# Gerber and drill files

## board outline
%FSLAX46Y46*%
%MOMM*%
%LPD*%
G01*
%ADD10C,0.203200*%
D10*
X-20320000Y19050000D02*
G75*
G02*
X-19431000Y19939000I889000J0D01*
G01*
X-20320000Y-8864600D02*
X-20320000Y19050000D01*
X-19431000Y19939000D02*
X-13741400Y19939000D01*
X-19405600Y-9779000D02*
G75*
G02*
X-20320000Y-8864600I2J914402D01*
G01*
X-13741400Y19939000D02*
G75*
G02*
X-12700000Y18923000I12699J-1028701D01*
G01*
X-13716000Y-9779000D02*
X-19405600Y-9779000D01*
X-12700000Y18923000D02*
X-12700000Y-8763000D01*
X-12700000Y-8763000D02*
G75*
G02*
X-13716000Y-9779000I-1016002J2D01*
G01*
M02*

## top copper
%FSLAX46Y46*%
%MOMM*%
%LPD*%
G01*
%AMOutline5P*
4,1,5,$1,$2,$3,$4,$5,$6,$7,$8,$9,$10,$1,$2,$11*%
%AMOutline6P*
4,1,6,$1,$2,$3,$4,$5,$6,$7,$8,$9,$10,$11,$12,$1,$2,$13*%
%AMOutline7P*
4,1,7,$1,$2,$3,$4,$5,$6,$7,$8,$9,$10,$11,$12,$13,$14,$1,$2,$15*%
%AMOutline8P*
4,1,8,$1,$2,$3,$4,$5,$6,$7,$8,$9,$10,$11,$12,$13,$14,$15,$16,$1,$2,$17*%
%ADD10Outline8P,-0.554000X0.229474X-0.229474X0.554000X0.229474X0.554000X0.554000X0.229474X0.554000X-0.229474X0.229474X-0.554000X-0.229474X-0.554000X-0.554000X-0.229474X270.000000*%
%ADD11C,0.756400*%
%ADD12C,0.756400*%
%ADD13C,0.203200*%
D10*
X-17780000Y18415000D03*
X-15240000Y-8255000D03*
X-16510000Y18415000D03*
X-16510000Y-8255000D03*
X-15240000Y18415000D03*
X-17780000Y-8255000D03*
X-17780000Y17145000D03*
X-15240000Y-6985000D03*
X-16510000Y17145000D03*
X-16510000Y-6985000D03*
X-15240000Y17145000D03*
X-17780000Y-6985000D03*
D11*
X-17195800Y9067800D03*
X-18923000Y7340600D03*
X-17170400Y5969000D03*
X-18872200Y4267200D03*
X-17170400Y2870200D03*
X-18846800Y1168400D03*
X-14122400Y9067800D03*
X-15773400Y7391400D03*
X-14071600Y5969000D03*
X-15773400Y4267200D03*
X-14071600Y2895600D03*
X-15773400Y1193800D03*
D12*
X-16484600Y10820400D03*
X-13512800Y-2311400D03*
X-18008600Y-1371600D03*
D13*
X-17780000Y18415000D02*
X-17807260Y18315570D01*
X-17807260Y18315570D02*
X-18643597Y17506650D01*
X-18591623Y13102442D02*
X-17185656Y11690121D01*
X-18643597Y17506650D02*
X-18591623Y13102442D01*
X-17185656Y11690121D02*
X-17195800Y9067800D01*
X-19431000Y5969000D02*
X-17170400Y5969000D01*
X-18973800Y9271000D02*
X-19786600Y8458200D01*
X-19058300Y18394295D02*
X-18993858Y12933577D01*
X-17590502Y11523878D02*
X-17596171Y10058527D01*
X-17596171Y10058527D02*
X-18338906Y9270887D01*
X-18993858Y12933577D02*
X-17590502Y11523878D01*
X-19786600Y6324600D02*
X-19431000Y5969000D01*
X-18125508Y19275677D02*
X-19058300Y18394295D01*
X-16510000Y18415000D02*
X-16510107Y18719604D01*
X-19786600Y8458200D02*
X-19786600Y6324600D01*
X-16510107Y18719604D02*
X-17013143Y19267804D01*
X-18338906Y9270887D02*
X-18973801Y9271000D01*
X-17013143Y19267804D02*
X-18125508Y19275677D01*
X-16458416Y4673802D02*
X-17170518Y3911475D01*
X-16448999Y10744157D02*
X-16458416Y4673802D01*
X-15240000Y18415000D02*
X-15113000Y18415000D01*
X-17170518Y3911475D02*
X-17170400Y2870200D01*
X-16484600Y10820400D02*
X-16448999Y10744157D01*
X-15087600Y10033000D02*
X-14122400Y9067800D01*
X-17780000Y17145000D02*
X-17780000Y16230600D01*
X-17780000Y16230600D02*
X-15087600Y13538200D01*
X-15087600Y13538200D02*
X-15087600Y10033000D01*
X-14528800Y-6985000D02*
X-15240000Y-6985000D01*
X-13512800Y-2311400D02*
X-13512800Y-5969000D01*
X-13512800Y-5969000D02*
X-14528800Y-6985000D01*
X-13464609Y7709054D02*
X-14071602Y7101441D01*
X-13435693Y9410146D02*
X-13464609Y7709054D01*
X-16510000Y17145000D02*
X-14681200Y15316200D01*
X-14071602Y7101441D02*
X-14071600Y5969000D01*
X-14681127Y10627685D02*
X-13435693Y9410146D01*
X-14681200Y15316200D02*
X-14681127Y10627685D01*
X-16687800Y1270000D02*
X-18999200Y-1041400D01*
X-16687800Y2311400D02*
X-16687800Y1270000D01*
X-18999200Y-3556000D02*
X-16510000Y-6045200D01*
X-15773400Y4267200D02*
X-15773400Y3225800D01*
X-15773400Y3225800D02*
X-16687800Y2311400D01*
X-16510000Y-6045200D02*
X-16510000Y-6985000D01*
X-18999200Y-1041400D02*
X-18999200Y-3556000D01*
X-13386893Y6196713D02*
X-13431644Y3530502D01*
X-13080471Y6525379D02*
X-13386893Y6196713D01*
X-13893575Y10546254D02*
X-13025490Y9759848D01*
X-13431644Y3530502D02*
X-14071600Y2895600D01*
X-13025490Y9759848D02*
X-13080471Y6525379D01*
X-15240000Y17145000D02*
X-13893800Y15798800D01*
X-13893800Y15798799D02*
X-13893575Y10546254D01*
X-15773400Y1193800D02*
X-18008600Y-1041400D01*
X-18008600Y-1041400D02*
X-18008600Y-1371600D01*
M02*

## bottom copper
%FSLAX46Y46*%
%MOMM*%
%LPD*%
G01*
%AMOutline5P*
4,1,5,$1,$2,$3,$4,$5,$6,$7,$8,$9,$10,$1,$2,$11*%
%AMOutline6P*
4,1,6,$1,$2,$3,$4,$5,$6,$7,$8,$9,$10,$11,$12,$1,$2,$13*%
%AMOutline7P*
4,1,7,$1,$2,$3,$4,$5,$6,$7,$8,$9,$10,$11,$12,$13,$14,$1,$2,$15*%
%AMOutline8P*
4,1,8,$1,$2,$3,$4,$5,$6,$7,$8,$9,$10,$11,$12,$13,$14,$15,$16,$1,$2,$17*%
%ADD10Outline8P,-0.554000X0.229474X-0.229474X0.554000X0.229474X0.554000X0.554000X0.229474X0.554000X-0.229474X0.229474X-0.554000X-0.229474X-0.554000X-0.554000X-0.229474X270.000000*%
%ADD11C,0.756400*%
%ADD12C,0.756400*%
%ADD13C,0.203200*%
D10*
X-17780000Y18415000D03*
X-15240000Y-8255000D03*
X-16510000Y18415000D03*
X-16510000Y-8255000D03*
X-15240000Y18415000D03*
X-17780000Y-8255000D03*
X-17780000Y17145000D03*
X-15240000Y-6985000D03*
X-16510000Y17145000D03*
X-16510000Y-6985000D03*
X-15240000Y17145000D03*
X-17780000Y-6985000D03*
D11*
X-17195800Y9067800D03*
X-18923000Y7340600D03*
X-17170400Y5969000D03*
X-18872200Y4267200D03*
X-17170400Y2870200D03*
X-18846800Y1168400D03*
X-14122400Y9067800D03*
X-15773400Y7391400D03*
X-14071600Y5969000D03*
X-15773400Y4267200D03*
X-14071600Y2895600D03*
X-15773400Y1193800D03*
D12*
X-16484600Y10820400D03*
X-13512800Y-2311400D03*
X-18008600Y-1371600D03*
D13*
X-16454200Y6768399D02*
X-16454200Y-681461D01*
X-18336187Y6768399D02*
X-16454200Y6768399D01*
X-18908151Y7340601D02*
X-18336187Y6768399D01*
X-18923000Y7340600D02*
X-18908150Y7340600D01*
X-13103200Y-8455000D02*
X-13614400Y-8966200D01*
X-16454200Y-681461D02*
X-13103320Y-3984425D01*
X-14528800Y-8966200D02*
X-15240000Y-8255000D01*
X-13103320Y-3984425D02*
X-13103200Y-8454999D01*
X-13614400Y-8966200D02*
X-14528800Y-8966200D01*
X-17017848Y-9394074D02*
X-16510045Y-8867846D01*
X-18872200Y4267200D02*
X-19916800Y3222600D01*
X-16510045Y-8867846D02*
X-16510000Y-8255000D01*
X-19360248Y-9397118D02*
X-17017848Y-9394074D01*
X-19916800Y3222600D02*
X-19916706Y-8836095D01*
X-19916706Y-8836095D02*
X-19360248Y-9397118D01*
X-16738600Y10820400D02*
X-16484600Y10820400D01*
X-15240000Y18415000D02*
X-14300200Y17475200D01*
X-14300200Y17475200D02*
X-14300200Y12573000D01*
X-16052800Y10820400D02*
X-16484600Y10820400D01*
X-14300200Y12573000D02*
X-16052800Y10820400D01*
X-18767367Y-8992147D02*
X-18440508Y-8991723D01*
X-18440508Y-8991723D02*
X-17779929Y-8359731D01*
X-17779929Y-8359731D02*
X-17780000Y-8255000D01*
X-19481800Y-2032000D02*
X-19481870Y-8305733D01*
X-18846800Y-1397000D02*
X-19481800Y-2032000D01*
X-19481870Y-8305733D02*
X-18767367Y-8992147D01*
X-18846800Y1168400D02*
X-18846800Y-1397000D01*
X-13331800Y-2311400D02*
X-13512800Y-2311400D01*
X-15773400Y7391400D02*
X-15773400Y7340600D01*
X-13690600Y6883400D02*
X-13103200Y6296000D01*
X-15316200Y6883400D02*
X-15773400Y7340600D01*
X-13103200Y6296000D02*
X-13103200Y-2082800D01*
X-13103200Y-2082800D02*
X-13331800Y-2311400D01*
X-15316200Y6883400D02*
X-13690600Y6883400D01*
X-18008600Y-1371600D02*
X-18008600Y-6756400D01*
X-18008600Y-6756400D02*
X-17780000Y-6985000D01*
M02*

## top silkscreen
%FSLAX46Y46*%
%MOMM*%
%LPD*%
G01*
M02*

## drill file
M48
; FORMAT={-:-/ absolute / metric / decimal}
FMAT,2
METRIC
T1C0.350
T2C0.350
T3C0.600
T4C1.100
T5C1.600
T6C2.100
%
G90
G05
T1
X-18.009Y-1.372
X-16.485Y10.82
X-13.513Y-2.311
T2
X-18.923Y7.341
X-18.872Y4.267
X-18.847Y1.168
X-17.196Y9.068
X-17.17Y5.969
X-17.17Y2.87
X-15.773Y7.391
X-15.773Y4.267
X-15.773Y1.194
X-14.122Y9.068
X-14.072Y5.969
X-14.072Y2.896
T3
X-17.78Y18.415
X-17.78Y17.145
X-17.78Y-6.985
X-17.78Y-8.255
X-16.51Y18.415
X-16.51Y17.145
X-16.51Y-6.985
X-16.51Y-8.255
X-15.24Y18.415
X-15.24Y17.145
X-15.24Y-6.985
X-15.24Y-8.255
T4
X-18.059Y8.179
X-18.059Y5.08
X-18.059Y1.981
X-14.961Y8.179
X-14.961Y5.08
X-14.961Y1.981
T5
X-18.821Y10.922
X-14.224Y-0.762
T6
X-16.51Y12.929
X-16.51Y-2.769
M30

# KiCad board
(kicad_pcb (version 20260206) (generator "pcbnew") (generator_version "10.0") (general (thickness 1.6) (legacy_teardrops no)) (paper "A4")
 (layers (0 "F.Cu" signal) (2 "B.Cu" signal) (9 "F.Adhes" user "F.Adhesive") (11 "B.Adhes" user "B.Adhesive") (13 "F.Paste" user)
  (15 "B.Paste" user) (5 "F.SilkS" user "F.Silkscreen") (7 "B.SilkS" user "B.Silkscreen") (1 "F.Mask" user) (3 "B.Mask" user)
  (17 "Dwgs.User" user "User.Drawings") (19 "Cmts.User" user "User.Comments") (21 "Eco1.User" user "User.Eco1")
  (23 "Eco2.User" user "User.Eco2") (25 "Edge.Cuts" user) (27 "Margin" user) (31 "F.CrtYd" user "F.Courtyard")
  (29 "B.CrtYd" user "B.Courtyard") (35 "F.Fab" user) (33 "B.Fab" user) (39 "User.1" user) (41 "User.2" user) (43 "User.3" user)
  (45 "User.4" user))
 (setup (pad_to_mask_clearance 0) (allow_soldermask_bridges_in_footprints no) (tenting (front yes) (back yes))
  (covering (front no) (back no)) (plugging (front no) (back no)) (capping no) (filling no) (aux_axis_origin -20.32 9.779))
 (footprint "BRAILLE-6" (layer "F.Cu") (at -16.51 -5.08)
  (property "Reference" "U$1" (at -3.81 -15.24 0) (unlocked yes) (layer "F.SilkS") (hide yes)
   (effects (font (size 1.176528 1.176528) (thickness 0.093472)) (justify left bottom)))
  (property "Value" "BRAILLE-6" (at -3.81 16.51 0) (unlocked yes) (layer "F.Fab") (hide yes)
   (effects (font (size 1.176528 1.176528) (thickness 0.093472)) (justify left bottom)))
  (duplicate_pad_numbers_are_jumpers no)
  (pad "P$1" thru_hole roundrect (at -1.27 -13.335 270) (size 1.108 1.108) (drill 0.6) (layers "*.Cu" "*.Mask") (remove_unused_layers no)
   (roundrect_rratio 0.25) (chamfer_ratio 0.2928932188) (chamfer top_left top_right bottom_left bottom_right) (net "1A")
   (solder_mask_margin 0.025) (thermal_bridge_angle 0))
  (pad "P$2" thru_hole roundrect (at 1.27 13.335 270) (size 1.108 1.108) (drill 0.6) (layers "*.Cu" "*.Mask") (remove_unused_layers no)
   (roundrect_rratio 0.25) (chamfer_ratio 0.2928932188) (chamfer top_left top_right bottom_left bottom_right) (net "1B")
   (solder_mask_margin 0.025) (thermal_bridge_angle 0))
  (pad "P$3" thru_hole roundrect (at 0 -13.335 270) (size 1.108 1.108) (drill 0.6) (layers "*.Cu" "*.Mask") (remove_unused_layers no)
   (roundrect_rratio 0.25) (chamfer_ratio 0.2928932188) (chamfer top_left top_right bottom_left bottom_right) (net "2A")
   (solder_mask_margin 0.025) (thermal_bridge_angle 0))
  (pad "P$4" thru_hole roundrect (at 0 13.335 270) (size 1.108 1.108) (drill 0.6) (layers "*.Cu" "*.Mask") (remove_unused_layers no)
   (roundrect_rratio 0.25) (chamfer_ratio 0.2928932188) (chamfer top_left top_right bottom_left bottom_right) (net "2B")
   (solder_mask_margin 0.025) (thermal_bridge_angle 0))
  (pad "P$5" thru_hole roundrect (at 1.27 -13.335 270) (size 1.108 1.108) (drill 0.6) (layers "*.Cu" "*.Mask") (remove_unused_layers no)
   (roundrect_rratio 0.25) (chamfer_ratio 0.2928932188) (chamfer top_left top_right bottom_left bottom_right) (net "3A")
   (solder_mask_margin 0.025) (thermal_bridge_angle 0))
  (pad "P$6" thru_hole roundrect (at -1.27 13.335 270) (size 1.108 1.108) (drill 0.6) (layers "*.Cu" "*.Mask") (remove_unused_layers no)
   (roundrect_rratio 0.25) (chamfer_ratio 0.2928932188) (chamfer top_left top_right bottom_left bottom_right) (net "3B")
   (solder_mask_margin 0.025) (thermal_bridge_angle 0))
  (pad "P$7" thru_hole roundrect (at -1.27 -12.065 270) (size 1.108 1.108) (drill 0.6) (layers "*.Cu" "*.Mask") (remove_unused_layers no)
   (roundrect_rratio 0.25) (chamfer_ratio 0.2928932188) (chamfer top_left top_right bottom_left bottom_right) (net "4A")
   (solder_mask_margin 0.025) (thermal_bridge_angle 0))
  (pad "P$8" thru_hole roundrect (at 1.27 12.065 270) (size 1.108 1.108) (drill 0.6) (layers "*.Cu" "*.Mask") (remove_unused_layers no)
   (roundrect_rratio 0.25) (chamfer_ratio 0.2928932188) (chamfer top_left top_right bottom_left bottom_right) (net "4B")
   (solder_mask_margin 0.025) (thermal_bridge_angle 0))
  (pad "P$9" thru_hole roundrect (at 0 -12.065 270) (size 1.108 1.108) (drill 0.6) (layers "*.Cu" "*.Mask") (remove_unused_layers no)
   (roundrect_rratio 0.25) (chamfer_ratio 0.2928932188) (chamfer top_left top_right bottom_left bottom_right) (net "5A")
   (solder_mask_margin 0.025) (thermal_bridge_angle 0))
  (pad "P$10" thru_hole roundrect (at 0 12.065 270) (size 1.108 1.108) (drill 0.6) (layers "*.Cu" "*.Mask") (remove_unused_layers no)
   (roundrect_rratio 0.25) (chamfer_ratio 0.2928932188) (chamfer top_left top_right bottom_left bottom_right) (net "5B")
   (solder_mask_margin 0.025) (thermal_bridge_angle 0))
  (pad "P$11" thru_hole roundrect (at 1.27 -12.065 270) (size 1.108 1.108) (drill 0.6) (layers "*.Cu" "*.Mask") (remove_unused_layers no)
   (roundrect_rratio 0.25) (chamfer_ratio 0.2928932188) (chamfer top_left top_right bottom_left bottom_right) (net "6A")
   (solder_mask_margin 0.025) (thermal_bridge_angle 0))
  (pad "P$12" thru_hole roundrect (at -1.27 12.065 270) (size 1.108 1.108) (drill 0.6) (layers "*.Cu" "*.Mask") (remove_unused_layers no)
   (roundrect_rratio 0.25) (chamfer_ratio 0.2928932188) (chamfer top_left top_right bottom_left bottom_right) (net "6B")
   (solder_mask_margin 0.025) (thermal_bridge_angle 0)))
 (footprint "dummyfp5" (layer "F.Cu") (at -14.9606 -1.9812)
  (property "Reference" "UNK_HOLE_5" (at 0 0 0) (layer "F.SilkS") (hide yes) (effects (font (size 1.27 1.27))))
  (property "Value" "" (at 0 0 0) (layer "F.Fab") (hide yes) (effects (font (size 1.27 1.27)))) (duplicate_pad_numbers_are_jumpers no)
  (pad "" np_thru_hole circle (at 0 0) (size 1.1 1.1) (drill 1.1) (layers "*.Cu" "*.Mask")))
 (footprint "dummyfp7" (layer "F.Cu") (at -16.51 2.7686)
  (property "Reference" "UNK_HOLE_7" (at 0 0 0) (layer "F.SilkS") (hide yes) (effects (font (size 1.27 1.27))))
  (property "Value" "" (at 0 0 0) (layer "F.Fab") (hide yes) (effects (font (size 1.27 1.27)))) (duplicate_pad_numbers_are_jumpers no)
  (pad "" np_thru_hole circle (at 0 0) (size 2.1 2.1) (drill 2.1) (layers "*.Cu" "*.Mask")))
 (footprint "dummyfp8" (layer "F.Cu") (at -18.8214 -10.922)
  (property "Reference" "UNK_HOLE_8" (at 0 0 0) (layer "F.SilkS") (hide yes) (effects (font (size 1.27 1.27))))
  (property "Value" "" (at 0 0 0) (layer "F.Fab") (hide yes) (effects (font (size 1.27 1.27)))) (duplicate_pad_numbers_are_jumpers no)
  (pad "" np_thru_hole circle (at 0 0) (size 1.6 1.6) (drill 1.6) (layers "*.Cu" "*.Mask")))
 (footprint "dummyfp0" (layer "F.Cu") (at -18.0594 -8.1788)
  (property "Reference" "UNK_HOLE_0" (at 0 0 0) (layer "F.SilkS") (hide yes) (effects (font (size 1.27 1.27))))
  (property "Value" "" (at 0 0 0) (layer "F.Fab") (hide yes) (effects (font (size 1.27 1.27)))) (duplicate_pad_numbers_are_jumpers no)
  (pad "" np_thru_hole circle (at 0 0) (size 1.1 1.1) (drill 1.1) (layers "*.Cu" "*.Mask")))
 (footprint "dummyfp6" (layer "F.Cu") (at -16.51 -12.9286)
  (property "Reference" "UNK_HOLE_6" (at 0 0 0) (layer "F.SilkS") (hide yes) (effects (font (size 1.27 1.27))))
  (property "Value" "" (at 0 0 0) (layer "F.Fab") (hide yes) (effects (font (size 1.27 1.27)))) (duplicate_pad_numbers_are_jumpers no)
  (pad "" np_thru_hole circle (at 0 0) (size 2.1 2.1) (drill 2.1) (layers "*.Cu" "*.Mask")))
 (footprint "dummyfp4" (layer "F.Cu") (at -18.0594 -1.9812)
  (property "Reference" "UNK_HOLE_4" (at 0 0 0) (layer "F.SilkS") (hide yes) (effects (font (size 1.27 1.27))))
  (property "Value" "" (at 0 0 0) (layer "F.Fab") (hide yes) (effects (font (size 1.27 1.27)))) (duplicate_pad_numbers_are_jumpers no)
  (pad "" np_thru_hole circle (at 0 0) (size 1.1 1.1) (drill 1.1) (layers "*.Cu" "*.Mask")))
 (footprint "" (layer "F.Cu") (at 0 0)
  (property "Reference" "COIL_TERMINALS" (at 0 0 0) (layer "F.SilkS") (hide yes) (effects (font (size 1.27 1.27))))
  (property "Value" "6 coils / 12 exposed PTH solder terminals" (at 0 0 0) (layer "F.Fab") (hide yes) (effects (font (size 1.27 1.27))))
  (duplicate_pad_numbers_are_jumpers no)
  (pad "1A" thru_hole circle (at -17.1958 -9.0678) (size 0.7564 0.7564) (drill 0.35) (layers "*.Cu" "*.Mask") (remove_unused_layers no)
   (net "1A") (solder_mask_margin 0.025))
  (pad "1B" thru_hole circle (at -18.923 -7.3406) (size 0.7564 0.7564) (drill 0.35) (layers "*.Cu" "*.Mask") (remove_unused_layers no)
   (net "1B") (solder_mask_margin 0.025))
  (pad "2A" thru_hole circle (at -17.1704 -5.969) (size 0.7564 0.7564) (drill 0.35) (layers "*.Cu" "*.Mask") (remove_unused_layers no)
   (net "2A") (solder_mask_margin 0.025))
  (pad "2B" thru_hole circle (at -18.8722 -4.2672) (size 0.7564 0.7564) (drill 0.35) (layers "*.Cu" "*.Mask") (remove_unused_layers no)
   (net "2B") (solder_mask_margin 0.025))
  (pad "3A" thru_hole circle (at -17.1704 -2.8702) (size 0.7564 0.7564) (drill 0.35) (layers "*.Cu" "*.Mask") (remove_unused_layers no)
   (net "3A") (solder_mask_margin 0.025))
  (pad "3B" thru_hole circle (at -18.8468 -1.1684) (size 0.7564 0.7564) (drill 0.35) (layers "*.Cu" "*.Mask") (remove_unused_layers no)
   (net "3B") (solder_mask_margin 0.025))
  (pad "4A" thru_hole circle (at -14.1224 -9.0678) (size 0.7564 0.7564) (drill 0.35) (layers "*.Cu" "*.Mask") (remove_unused_layers no)
   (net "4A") (solder_mask_margin 0.025))
  (pad "4B" thru_hole circle (at -15.7734 -7.3914) (size 0.7564 0.7564) (drill 0.35) (layers "*.Cu" "*.Mask") (remove_unused_layers no)
   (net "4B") (solder_mask_margin 0.025))
  (pad "5A" thru_hole circle (at -14.0716 -5.969) (size 0.7564 0.7564) (drill 0.35) (layers "*.Cu" "*.Mask") (remove_unused_layers no)
   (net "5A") (solder_mask_margin 0.025))
  (pad "5B" thru_hole circle (at -15.7734 -4.2672) (size 0.7564 0.7564) (drill 0.35) (layers "*.Cu" "*.Mask") (remove_unused_layers no)
   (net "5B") (solder_mask_margin 0.025))
  (pad "6A" thru_hole circle (at -14.0716 -2.8956) (size 0.7564 0.7564) (drill 0.35) (layers "*.Cu" "*.Mask") (remove_unused_layers no)
   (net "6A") (solder_mask_margin 0.025))
  (pad "6B" thru_hole circle (at -15.7734 -1.1938) (size 0.7564 0.7564) (drill 0.35) (layers "*.Cu" "*.Mask") (remove_unused_layers no)
   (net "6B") (solder_mask_margin 0.025)))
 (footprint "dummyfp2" (layer "F.Cu") (at -18.0594 -5.08)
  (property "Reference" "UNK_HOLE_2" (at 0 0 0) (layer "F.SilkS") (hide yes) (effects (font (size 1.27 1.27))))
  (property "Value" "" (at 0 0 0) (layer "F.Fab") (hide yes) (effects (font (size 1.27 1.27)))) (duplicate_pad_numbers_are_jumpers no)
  (pad "" np_thru_hole circle (at 0 0) (size 1.1 1.1) (drill 1.1) (layers "*.Cu" "*.Mask")))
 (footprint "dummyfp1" (layer "F.Cu") (at -14.9606 -8.1788)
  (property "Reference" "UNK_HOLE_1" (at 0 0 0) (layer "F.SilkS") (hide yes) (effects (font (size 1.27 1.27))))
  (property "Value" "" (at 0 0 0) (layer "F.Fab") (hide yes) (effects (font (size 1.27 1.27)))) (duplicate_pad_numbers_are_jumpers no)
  (pad "" np_thru_hole circle (at 0 0) (size 1.1 1.1) (drill 1.1) (layers "*.Cu" "*.Mask")))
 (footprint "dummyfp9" (layer "F.Cu") (at -14.224 0.762)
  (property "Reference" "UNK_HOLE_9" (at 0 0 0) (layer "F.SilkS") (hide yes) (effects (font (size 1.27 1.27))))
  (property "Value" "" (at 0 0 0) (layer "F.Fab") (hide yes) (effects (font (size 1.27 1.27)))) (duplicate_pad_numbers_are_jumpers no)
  (pad "" np_thru_hole circle (at 0 0) (size 1.6 1.6) (drill 1.6) (layers "*.Cu" "*.Mask")))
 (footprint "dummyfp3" (layer "F.Cu") (at -14.9606 -5.08)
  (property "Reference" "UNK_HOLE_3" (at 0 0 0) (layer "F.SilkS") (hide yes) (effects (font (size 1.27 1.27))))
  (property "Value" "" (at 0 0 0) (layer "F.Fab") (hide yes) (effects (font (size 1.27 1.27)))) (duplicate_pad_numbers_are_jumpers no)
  (pad "" np_thru_hole circle (at 0 0) (size 1.1 1.1) (drill 1.1) (layers "*.Cu" "*.Mask")))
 (gr_arc (start -20.32 -19.05) (mid -20.059618 -19.678618) (end -19.431 -19.939) (stroke (width 0.2032) (type solid)) (layer "Edge.Cuts"))
 (gr_line (start -20.32 8.8646) (end -20.32 -19.05) (stroke (width 0.2032) (type solid)) (layer "Edge.Cuts"))
 (gr_line (start -19.431 -19.939) (end -13.7414 -19.939) (stroke (width 0.2032) (type solid)) (layer "Edge.Cuts"))
 (gr_arc (start -19.4056 9.779) (mid -20.052178 9.511178) (end -20.32 8.8646) (stroke (width 0.2032) (type solid)) (layer "Edge.Cuts"))
 (gr_arc (start -13.7414 -19.939) (mid -13.01028 -19.646681) (end -12.7 -18.923) (stroke (width 0.2032) (type solid)) (layer "Edge.Cuts"))
 (gr_line (start -13.716 9.779) (end -19.4056 9.779) (stroke (width 0.2032) (type solid)) (layer "Edge.Cuts"))
 (gr_line (start -12.7 -18.923) (end -12.7 8.763) (stroke (width 0.2032) (type solid)) (layer "Edge.Cuts"))
 (gr_arc (start -12.7 8.763) (mid -12.99758 9.48142) (end -13.716 9.779) (stroke (width 0.2032) (type solid)) (layer "Edge.Cuts"))
 (segment (start -17.78 -18.415) (end -17.80726 -18.31557) (width 0.2032) (layer "F.Cu") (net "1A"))
 (segment (start -17.80726 -18.31557) (end -18.643597 -17.50665) (width 0.2032) (layer "F.Cu") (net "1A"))
 (segment (start -18.591623 -13.102442) (end -17.185656 -11.690121) (width 0.2032) (layer "F.Cu") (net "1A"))
 (segment (start -18.643597 -17.50665) (end -18.591623 -13.102442) (width 0.2032) (layer "F.Cu") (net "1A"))
 (segment (start -17.185656 -11.690121) (end -17.1958 -9.0678) (width 0.2032) (layer "F.Cu") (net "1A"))
 (segment (start -16.4542 -6.768399) (end -16.4542 0.681461) (width 0.2032) (layer "B.Cu") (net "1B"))
 (segment (start -18.336187 -6.768399) (end -16.4542 -6.768399) (width 0.2032) (layer "B.Cu") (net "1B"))
 (segment (start -18.908151 -7.340601) (end -18.336187 -6.768399) (width 0.2032) (layer "B.Cu") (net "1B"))
 (segment (start -18.923 -7.3406) (end -18.90815 -7.3406) (width 0.2032) (layer "B.Cu") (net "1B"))
 (segment (start -13.1032 8.455) (end -13.6144 8.9662) (width 0.2032) (layer "B.Cu") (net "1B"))
 (segment (start -16.4542 0.681461) (end -13.10332 3.984425) (width 0.2032) (layer "B.Cu") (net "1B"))
 (segment (start -14.5288 8.9662) (end -15.24 8.255) (width 0.2032) (layer "B.Cu") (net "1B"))
 (segment (start -13.10332 3.984425) (end -13.1032 8.454999) (width 0.2032) (layer "B.Cu") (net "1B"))
 (segment (start -13.6144 8.9662) (end -14.5288 8.9662) (width 0.2032) (layer "B.Cu") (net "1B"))
 (segment (start -19.431 -5.969) (end -17.1704 -5.969) (width 0.2032) (layer "F.Cu") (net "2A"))
 (segment (start -18.9738 -9.271) (end -19.7866 -8.4582) (width 0.2032) (layer "F.Cu") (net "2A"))
 (segment (start -19.0583 -18.394295) (end -18.993858 -12.933577) (width 0.2032) (layer "F.Cu") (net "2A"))
 (segment (start -17.590502 -11.523878) (end -17.596171 -10.058527) (width 0.2032) (layer "F.Cu") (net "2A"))
 (segment (start -17.596171 -10.058527) (end -18.338906 -9.270887) (width 0.2032) (layer "F.Cu") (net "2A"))
 (segment (start -18.993858 -12.933577) (end -17.590502 -11.523878) (width 0.2032) (layer "F.Cu") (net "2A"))
 (segment (start -19.7866 -6.3246) (end -19.431 -5.969) (width 0.2032) (layer "F.Cu") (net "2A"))
 (segment (start -18.125508 -19.275677) (end -19.0583 -18.394295) (width 0.2032) (layer "F.Cu") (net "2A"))
 (segment (start -16.51 -18.415) (end -16.510107 -18.719604) (width 0.2032) (layer "F.Cu") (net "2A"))
 (segment (start -19.7866 -8.4582) (end -19.7866 -6.3246) (width 0.2032) (layer "F.Cu") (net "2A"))
 (segment (start -16.510107 -18.719604) (end -17.013143 -19.267804) (width 0.2032) (layer "F.Cu") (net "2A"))
 (segment (start -18.338906 -9.270887) (end -18.973801 -9.271) (width 0.2032) (layer "F.Cu") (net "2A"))
 (segment (start -17.013143 -19.267804) (end -18.125508 -19.275677) (width 0.2032) (layer "F.Cu") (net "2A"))
 (segment (start -17.017848 9.394074) (end -16.510045 8.867846) (width 0.2032) (layer "B.Cu") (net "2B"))
 (segment (start -18.8722 -4.2672) (end -19.9168 -3.2226) (width 0.2032) (layer "B.Cu") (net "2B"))
 (segment (start -16.510045 8.867846) (end -16.51 8.255) (width 0.2032) (layer "B.Cu") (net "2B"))
 (segment (start -19.360248 9.397118) (end -17.017848 9.394074) (width 0.2032) (layer "B.Cu") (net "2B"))
 (segment (start -19.9168 -3.2226) (end -19.916706 8.836095) (width 0.2032) (layer "B.Cu") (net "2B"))
 (segment (start -19.916706 8.836095) (end -19.360248 9.397118) (width 0.2032) (layer "B.Cu") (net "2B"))
 (segment (start -16.458416 -4.673802) (end -17.170518 -3.911475) (width 0.2032) (layer "F.Cu") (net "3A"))
 (segment (start -16.448999 -10.744157) (end -16.458416 -4.673802) (width 0.2032) (layer "F.Cu") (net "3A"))
 (segment (start -15.24 -18.415) (end -15.113 -18.415) (width 0.2032) (layer "F.Cu") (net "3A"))
 (segment (start -17.170518 -3.911475) (end -17.1704 -2.8702) (width 0.2032) (layer "F.Cu") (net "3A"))
 (segment (start -16.4846 -10.8204) (end -16.448999 -10.744157) (width 0.2032) (layer "F.Cu") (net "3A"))
 (via (at -16.4846 -10.8204) (size 0.7564) (drill 0.35) (layers "F.Cu" "B.Cu") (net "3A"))
 (segment (start -16.7386 -10.8204) (end -16.4846 -10.8204) (width 0.2032) (layer "B.Cu") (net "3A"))
 (segment (start -15.24 -18.415) (end -14.3002 -17.4752) (width 0.2032) (layer "B.Cu") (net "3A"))
 (segment (start -14.3002 -17.4752) (end -14.3002 -12.573) (width 0.2032) (layer "B.Cu") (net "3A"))
 (segment (start -16.0528 -10.8204) (end -16.4846 -10.8204) (width 0.2032) (layer "B.Cu") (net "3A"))
 (segment (start -14.3002 -12.573) (end -16.0528 -10.8204) (width 0.2032) (layer "B.Cu") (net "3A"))
 (segment (start -18.767367 8.992147) (end -18.440508 8.991723) (width 0.2032) (layer "B.Cu") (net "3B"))
 (segment (start -18.440508 8.991723) (end -17.779929 8.359731) (width 0.2032) (layer "B.Cu") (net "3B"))
 (segment (start -17.779929 8.359731) (end -17.78 8.255) (width 0.2032) (layer "B.Cu") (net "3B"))
 (segment (start -19.4818 2.032) (end -19.48187 8.305733) (width 0.2032) (layer "B.Cu") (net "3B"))
 (segment (start -18.8468 1.397) (end -19.4818 2.032) (width 0.2032) (layer "B.Cu") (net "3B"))
 (segment (start -19.48187 8.305733) (end -18.767367 8.992147) (width 0.2032) (layer "B.Cu") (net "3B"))
 (segment (start -18.8468 -1.1684) (end -18.8468 1.397) (width 0.2032) (layer "B.Cu") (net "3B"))
 (segment (start -15.0876 -10.033) (end -14.1224 -9.0678) (width 0.2032) (layer "F.Cu") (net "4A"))
 (segment (start -17.78 -17.145) (end -17.78 -16.2306) (width 0.2032) (layer "F.Cu") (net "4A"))
 (segment (start -17.78 -16.2306) (end -15.0876 -13.5382) (width 0.2032) (layer "F.Cu") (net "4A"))
 (segment (start -15.0876 -13.5382) (end -15.0876 -10.033) (width 0.2032) (layer "F.Cu") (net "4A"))
 (segment (start -14.5288 6.985) (end -15.24 6.985) (width 0.2032) (layer "F.Cu") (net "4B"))
 (segment (start -13.5128 2.3114) (end -13.5128 5.969) (width 0.2032) (layer "F.Cu") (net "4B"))
 (segment (start -13.5128 5.969) (end -14.5288 6.985) (width 0.2032) (layer "F.Cu") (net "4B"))
 (via (at -13.5128 2.3114) (size 0.7564) (drill 0.35) (layers "F.Cu" "B.Cu") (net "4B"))
 (segment (start -13.3318 2.3114) (end -13.5128 2.3114) (width 0.2032) (layer "B.Cu") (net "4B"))
 (segment (start -15.7734 -7.3914) (end -15.7734 -7.3406) (width 0.2032) (layer "B.Cu") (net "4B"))
 (segment (start -13.6906 -6.8834) (end -13.1032 -6.296) (width 0.2032) (layer "B.Cu") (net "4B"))
 (segment (start -15.3162 -6.8834) (end -15.7734 -7.3406) (width 0.2032) (layer "B.Cu") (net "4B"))
 (segment (start -13.1032 -6.296) (end -13.1032 2.0828) (width 0.2032) (layer "B.Cu") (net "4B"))
 (segment (start -13.1032 2.0828) (end -13.3318 2.3114) (width 0.2032) (layer "B.Cu") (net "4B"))
 (segment (start -15.3162 -6.8834) (end -13.6906 -6.8834) (width 0.2032) (layer "B.Cu") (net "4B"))
 (segment (start -13.464609 -7.709054) (end -14.071602 -7.101441) (width 0.2032) (layer "F.Cu") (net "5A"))
 (segment (start -13.435693 -9.410146) (end -13.464609 -7.709054) (width 0.2032) (layer "F.Cu") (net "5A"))
 (segment (start -16.51 -17.145) (end -14.6812 -15.3162) (width 0.2032) (layer "F.Cu") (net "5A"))
 (segment (start -14.071602 -7.101441) (end -14.0716 -5.969) (width 0.2032) (layer "F.Cu") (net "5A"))
 (segment (start -14.681127 -10.627685) (end -13.435693 -9.410146) (width 0.2032) (layer "F.Cu") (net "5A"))
 (segment (start -14.6812 -15.3162) (end -14.681127 -10.627685) (width 0.2032) (layer "F.Cu") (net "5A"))
 (segment (start -16.6878 -1.27) (end -18.9992 1.0414) (width 0.2032) (layer "F.Cu") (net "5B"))
 (segment (start -16.6878 -2.3114) (end -16.6878 -1.27) (width 0.2032) (layer "F.Cu") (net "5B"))
 (segment (start -18.9992 3.556) (end -16.51 6.0452) (width 0.2032) (layer "F.Cu") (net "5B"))
 (segment (start -15.7734 -4.2672) (end -15.7734 -3.2258) (width 0.2032) (layer "F.Cu") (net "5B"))
 (segment (start -15.7734 -3.2258) (end -16.6878 -2.3114) (width 0.2032) (layer "F.Cu") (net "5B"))
 (segment (start -16.51 6.0452) (end -16.51 6.985) (width 0.2032) (layer "F.Cu") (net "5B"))
 (segment (start -18.9992 1.0414) (end -18.9992 3.556) (width 0.2032) (layer "F.Cu") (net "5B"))
 (segment (start -13.386893 -6.196713) (end -13.431644 -3.530502) (width 0.2032) (layer "F.Cu") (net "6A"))
 (segment (start -13.080471 -6.525379) (end -13.386893 -6.196713) (width 0.2032) (layer "F.Cu") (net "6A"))
 (segment (start -13.893575 -10.546254) (end -13.02549 -9.759848) (width 0.2032) (layer "F.Cu") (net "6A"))
 (segment (start -13.431644 -3.530502) (end -14.0716 -2.8956) (width 0.2032) (layer "F.Cu") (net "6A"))
 (segment (start -13.02549 -9.759848) (end -13.080471 -6.525379) (width 0.2032) (layer "F.Cu") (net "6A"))
 (segment (start -15.24 -17.145) (end -13.8938 -15.7988) (width 0.2032) (layer "F.Cu") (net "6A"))
 (segment (start -13.8938 -15.798799) (end -13.893575 -10.546254) (width 0.2032) (layer "F.Cu") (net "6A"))
 (segment (start -15.7734 -1.1938) (end -18.0086 1.0414) (width 0.2032) (layer "F.Cu") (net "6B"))
 (segment (start -18.0086 1.0414) (end -18.0086 1.3716) (width 0.2032) (layer "F.Cu") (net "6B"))
 (via (at -18.0086 1.3716) (size 0.7564) (drill 0.35) (layers "F.Cu" "B.Cu") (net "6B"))
 (segment (start -18.0086 1.3716) (end -18.0086 6.7564) (width 0.2032) (layer "B.Cu") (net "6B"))
 (segment (start -18.0086 6.7564) (end -17.78 6.985) (width 0.2032) (layer "B.Cu") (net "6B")))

